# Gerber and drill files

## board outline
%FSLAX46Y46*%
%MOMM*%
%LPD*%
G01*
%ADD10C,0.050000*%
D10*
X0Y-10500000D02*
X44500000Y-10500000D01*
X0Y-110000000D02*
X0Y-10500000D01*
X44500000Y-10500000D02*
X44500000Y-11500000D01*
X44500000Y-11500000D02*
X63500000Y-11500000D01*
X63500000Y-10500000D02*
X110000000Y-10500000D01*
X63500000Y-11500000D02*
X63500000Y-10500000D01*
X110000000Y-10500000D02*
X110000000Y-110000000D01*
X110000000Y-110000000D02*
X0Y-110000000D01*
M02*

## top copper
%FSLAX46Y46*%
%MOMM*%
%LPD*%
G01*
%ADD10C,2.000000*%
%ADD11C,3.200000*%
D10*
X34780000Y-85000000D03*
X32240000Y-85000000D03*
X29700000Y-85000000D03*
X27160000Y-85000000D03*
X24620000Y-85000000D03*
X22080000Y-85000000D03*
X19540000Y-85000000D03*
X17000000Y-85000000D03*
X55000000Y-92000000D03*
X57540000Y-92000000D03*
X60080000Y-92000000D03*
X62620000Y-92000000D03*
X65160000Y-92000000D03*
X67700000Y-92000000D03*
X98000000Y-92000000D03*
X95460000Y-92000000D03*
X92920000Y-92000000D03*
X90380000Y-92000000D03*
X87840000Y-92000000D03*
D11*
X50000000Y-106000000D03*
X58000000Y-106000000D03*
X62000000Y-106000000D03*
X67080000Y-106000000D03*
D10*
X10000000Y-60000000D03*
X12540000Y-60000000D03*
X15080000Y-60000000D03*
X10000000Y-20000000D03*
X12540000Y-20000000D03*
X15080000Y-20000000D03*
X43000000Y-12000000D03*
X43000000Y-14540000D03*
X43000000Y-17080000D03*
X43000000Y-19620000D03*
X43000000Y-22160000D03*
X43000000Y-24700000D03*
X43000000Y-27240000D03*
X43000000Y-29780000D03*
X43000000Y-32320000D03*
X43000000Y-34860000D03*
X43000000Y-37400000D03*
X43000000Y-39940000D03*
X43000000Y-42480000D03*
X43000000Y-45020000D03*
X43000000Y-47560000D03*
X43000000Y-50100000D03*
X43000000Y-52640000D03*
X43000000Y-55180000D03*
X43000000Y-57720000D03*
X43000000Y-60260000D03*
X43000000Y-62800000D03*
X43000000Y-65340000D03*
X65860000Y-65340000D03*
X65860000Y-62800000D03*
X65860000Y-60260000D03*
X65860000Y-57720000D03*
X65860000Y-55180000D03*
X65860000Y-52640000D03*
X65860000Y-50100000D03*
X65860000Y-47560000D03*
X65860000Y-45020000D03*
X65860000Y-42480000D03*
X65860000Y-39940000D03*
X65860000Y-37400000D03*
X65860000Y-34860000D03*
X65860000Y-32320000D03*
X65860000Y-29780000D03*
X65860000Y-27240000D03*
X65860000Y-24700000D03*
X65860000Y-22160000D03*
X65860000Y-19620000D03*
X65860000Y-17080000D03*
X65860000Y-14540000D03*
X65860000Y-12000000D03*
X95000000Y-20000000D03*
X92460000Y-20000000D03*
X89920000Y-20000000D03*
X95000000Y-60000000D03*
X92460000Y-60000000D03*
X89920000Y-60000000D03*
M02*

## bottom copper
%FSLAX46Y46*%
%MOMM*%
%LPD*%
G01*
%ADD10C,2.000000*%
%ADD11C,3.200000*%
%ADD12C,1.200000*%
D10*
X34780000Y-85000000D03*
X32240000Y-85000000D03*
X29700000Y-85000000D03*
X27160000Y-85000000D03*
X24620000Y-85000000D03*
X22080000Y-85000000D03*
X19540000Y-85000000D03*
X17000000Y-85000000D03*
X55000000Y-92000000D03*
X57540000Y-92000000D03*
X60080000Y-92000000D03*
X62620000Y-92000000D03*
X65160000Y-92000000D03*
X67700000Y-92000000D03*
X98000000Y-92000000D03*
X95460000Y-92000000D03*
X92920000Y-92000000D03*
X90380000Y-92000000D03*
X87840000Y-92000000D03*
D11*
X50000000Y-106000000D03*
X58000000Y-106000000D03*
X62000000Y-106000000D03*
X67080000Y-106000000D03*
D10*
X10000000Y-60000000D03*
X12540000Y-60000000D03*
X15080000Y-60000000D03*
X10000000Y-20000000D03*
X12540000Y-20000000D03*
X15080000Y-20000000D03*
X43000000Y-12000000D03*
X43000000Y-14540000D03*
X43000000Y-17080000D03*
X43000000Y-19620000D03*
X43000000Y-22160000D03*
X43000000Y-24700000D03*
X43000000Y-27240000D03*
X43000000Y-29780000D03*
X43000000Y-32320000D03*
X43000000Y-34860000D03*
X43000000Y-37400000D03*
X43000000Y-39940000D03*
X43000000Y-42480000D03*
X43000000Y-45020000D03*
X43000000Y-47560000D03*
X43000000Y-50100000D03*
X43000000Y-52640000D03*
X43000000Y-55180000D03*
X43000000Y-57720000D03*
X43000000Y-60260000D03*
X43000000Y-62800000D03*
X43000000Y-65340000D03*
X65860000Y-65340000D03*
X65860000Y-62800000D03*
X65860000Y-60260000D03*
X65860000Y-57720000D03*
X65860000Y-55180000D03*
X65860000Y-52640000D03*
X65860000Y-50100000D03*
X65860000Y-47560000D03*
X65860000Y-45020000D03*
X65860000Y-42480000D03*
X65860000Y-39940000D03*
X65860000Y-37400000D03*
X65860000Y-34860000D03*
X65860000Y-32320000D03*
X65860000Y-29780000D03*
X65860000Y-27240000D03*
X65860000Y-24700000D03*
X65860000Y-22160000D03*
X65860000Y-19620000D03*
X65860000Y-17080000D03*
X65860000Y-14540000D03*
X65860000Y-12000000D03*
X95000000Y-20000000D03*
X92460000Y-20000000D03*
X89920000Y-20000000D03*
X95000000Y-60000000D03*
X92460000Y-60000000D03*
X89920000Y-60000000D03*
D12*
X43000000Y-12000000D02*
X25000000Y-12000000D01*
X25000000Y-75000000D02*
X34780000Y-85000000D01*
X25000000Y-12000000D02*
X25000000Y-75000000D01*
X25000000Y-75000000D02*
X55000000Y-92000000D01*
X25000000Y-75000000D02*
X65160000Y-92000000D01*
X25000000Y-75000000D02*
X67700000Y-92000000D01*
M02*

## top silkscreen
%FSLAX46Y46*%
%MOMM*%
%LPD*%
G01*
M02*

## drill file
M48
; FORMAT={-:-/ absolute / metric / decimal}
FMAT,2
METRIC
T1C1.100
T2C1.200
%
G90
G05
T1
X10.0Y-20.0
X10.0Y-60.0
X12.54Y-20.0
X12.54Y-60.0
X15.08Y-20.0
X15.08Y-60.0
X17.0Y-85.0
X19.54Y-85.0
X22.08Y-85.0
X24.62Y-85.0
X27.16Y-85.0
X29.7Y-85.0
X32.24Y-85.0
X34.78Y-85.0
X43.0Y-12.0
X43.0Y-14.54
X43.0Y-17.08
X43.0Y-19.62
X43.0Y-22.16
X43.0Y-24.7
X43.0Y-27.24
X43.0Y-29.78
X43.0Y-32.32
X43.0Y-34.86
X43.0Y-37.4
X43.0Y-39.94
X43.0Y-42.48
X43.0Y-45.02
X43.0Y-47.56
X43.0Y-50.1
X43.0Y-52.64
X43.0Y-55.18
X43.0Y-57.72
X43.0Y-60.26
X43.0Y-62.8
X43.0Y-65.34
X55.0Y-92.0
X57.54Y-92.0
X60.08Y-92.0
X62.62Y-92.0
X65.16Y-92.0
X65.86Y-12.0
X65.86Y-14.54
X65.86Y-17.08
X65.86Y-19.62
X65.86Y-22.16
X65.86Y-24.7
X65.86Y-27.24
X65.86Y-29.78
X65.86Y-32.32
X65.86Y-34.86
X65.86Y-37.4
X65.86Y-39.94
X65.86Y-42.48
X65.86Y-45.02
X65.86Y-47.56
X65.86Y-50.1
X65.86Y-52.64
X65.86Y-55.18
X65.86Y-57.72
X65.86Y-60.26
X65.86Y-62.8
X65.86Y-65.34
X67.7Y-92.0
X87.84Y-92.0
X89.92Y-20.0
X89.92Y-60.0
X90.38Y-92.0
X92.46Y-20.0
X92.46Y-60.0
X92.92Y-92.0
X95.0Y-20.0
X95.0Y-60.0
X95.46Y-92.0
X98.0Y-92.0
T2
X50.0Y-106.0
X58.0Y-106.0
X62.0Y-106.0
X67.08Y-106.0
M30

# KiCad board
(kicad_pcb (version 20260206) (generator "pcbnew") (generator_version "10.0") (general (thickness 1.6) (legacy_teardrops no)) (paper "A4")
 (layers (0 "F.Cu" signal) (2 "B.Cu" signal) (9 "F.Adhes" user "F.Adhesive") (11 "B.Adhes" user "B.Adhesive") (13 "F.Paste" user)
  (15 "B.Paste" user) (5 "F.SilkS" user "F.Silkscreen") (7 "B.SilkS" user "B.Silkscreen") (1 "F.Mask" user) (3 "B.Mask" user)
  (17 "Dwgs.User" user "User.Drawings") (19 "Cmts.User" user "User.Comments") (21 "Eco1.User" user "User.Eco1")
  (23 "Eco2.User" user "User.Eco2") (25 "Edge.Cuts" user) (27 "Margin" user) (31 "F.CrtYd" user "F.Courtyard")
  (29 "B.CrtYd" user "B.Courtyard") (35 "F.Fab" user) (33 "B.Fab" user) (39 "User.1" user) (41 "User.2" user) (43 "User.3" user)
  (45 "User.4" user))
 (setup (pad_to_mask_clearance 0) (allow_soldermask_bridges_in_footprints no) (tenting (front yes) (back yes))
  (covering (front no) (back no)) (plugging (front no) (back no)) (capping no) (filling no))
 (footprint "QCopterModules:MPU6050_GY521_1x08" (layer "F.Cu") (at 34.78 85 -90)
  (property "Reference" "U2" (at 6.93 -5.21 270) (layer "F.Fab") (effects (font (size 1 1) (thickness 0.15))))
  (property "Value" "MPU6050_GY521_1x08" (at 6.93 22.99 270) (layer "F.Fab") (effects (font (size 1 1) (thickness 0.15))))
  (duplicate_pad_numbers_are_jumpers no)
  (pad "1" thru_hole circle (at 0 0 270) (size 2 2) (drill 1.1) (layers "*.Cu" "*.Mask") (remove_unused_layers no) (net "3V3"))
  (pad "2" thru_hole circle (at 0 2.54 270) (size 2 2) (drill 1.1) (layers "*.Cu" "*.Mask") (remove_unused_layers no) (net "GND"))
  (pad "3" thru_hole circle (at 0 5.08 270) (size 2 2) (drill 1.1) (layers "*.Cu" "*.Mask") (remove_unused_layers no) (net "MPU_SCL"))
  (pad "4" thru_hole circle (at 0 7.62 270) (size 2 2) (drill 1.1) (layers "*.Cu" "*.Mask") (remove_unused_layers no) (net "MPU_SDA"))
  (pad "5" thru_hole circle (at 0 10.16 270) (size 2 2) (drill 1.1) (layers "*.Cu" "*.Mask") (remove_unused_layers no)
   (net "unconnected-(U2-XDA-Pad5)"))
  (pad "6" thru_hole circle (at 0 12.7 270) (size 2 2) (drill 1.1) (layers "*.Cu" "*.Mask") (remove_unused_layers no)
   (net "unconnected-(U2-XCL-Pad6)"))
  (pad "7" thru_hole circle (at 0 15.24 270) (size 2 2) (drill 1.1) (layers "*.Cu" "*.Mask") (remove_unused_layers no) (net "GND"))
  (pad "8" thru_hole circle (at 0 17.78 270) (size 2 2) (drill 1.1) (layers "*.Cu" "*.Mask") (remove_unused_layers no) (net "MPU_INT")))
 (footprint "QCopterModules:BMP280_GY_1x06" (layer "F.Cu") (at 55 92 90)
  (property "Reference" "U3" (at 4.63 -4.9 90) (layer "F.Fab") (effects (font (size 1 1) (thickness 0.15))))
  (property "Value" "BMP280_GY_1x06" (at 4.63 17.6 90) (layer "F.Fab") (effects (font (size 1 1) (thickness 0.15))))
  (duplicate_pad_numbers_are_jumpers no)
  (pad "1" thru_hole circle (at 0 0 90) (size 2 2) (drill 1.1) (layers "*.Cu" "*.Mask") (remove_unused_layers no) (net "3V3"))
  (pad "2" thru_hole circle (at 0 2.54 90) (size 2 2) (drill 1.1) (layers "*.Cu" "*.Mask") (remove_unused_layers no) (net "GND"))
  (pad "3" thru_hole circle (at 0 5.08 90) (size 2 2) (drill 1.1) (layers "*.Cu" "*.Mask") (remove_unused_layers no) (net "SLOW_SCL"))
  (pad "4" thru_hole circle (at 0 7.62 90) (size 2 2) (drill 1.1) (layers "*.Cu" "*.Mask") (remove_unused_layers no) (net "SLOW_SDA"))
  (pad "5" thru_hole circle (at 0 10.16 90) (size 2 2) (drill 1.1) (layers "*.Cu" "*.Mask") (remove_unused_layers no) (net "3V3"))
  (pad "6" thru_hole circle (at 0 12.7 90) (size 2 2) (drill 1.1) (layers "*.Cu" "*.Mask") (remove_unused_layers no) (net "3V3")))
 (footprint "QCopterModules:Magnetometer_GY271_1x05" (layer "F.Cu") (at 98 92 -90)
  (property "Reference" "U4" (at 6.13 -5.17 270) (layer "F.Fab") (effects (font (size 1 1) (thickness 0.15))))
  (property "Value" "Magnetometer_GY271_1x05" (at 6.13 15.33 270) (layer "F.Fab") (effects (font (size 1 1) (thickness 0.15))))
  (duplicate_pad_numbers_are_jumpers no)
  (pad "1" thru_hole circle (at 0 0 270) (size 2 2) (drill 1.1) (layers "*.Cu" "*.Mask") (remove_unused_layers no) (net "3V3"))
  (pad "2" thru_hole circle (at 0 2.54 270) (size 2 2) (drill 1.1) (layers "*.Cu" "*.Mask") (remove_unused_layers no) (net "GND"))
  (pad "3" thru_hole circle (at 0 5.08 270) (size 2 2) (drill 1.1) (layers "*.Cu" "*.Mask") (remove_unused_layers no) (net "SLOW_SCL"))
  (pad "4" thru_hole circle (at 0 7.62 270) (size 2 2) (drill 1.1) (layers "*.Cu" "*.Mask") (remove_unused_layers no) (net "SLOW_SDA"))
  (pad "5" thru_hole circle (at 0 10.16 270) (size 2 2) (drill 1.1) (layers "*.Cu" "*.Mask") (remove_unused_layers no) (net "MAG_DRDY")))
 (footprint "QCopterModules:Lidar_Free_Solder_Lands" (layer "F.Cu") (at 50 106)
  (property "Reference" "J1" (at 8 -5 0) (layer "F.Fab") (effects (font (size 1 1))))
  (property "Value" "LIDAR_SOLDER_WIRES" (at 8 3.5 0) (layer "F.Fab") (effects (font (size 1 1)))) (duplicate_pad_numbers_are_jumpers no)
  (pad "1" thru_hole circle (at 0 0) (size 3.2 3.2) (drill 1.2) (layers "*.Cu" "*.Mask") (remove_unused_layers no) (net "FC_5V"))
  (pad "2" thru_hole circle (at 8 0) (size 3.2 3.2) (drill 1.2) (layers "*.Cu" "*.Mask") (remove_unused_layers no) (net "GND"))
  (pad "3" thru_hole circle (at 12 0) (size 3.2 3.2) (drill 1.2) (layers "*.Cu" "*.Mask") (remove_unused_layers no) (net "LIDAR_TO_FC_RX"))
  (pad "4" thru_hole circle (at 17.08 0) (size 3.2 3.2) (drill 1.2) (layers "*.Cu" "*.Mask") (remove_unused_layers no)
   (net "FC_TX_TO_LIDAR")))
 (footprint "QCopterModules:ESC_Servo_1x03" (layer "F.Cu") (at 10 60 90)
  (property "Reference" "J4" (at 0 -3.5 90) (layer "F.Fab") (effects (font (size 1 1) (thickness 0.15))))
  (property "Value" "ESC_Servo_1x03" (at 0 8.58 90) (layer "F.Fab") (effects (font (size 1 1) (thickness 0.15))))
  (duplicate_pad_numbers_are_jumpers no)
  (pad "1" thru_hole circle (at 0 0 90) (size 2 2) (drill 1.1) (layers "*.Cu" "*.Mask") (remove_unused_layers no) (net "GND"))
  (pad "2" thru_hole circle (at 0 2.54 90) (size 2 2) (drill 1.1) (layers "*.Cu" "*.Mask") (remove_unused_layers no) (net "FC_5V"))
  (pad "3" thru_hole circle (at 0 5.08 90) (size 2 2) (drill 1.1) (layers "*.Cu" "*.Mask") (remove_unused_layers no) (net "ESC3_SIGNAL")))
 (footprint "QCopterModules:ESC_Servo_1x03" (layer "F.Cu") (at 10 20 90)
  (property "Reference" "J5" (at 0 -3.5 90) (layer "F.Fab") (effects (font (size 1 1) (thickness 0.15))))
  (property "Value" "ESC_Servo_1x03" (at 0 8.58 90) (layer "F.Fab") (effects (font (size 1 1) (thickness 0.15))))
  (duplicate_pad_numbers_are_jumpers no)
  (pad "1" thru_hole circle (at 0 0 90) (size 2 2) (drill 1.1) (layers "*.Cu" "*.Mask") (remove_unused_layers no) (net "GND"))
  (pad "2" thru_hole circle (at 0 2.54 90) (size 2 2) (drill 1.1) (layers "*.Cu" "*.Mask") (remove_unused_layers no)
   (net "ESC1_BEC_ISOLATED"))
  (pad "3" thru_hole circle (at 0 5.08 90) (size 2 2) (drill 1.1) (layers "*.Cu" "*.Mask") (remove_unused_layers no) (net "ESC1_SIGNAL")))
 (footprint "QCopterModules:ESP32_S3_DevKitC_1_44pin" (layer "F.Cu") (at 43 12)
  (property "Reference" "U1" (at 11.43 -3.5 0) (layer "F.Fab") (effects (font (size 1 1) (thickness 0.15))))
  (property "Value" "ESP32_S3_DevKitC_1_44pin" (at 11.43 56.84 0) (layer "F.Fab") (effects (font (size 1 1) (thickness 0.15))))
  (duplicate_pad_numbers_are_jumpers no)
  (pad "1" thru_hole circle (at 0 0) (size 2 2) (drill 1.1) (layers "*.Cu" "*.Mask") (remove_unused_layers no) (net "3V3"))
  (pad "2" thru_hole circle (at 0 2.54) (size 2 2) (drill 1.1) (layers "*.Cu" "*.Mask") (remove_unused_layers no))
  (pad "3" thru_hole circle (at 0 5.08) (size 2 2) (drill 1.1) (layers "*.Cu" "*.Mask") (remove_unused_layers no)
   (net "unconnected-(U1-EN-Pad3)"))
  (pad "4" thru_hole circle (at 0 7.62) (size 2 2) (drill 1.1) (layers "*.Cu" "*.Mask") (remove_unused_layers no) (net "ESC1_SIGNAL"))
  (pad "5" thru_hole circle (at 0 10.16) (size 2 2) (drill 1.1) (layers "*.Cu" "*.Mask") (remove_unused_layers no)
   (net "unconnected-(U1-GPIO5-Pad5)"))
  (pad "6" thru_hole circle (at 0 12.7) (size 2 2) (drill 1.1) (layers "*.Cu" "*.Mask") (remove_unused_layers no)
   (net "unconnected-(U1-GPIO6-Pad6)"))
  (pad "7" thru_hole circle (at 0 15.24) (size 2 2) (drill 1.1) (layers "*.Cu" "*.Mask") (remove_unused_layers no)
   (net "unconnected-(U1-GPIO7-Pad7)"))
  (pad "8" thru_hole circle (at 0 17.78) (size 2 2) (drill 1.1) (layers "*.Cu" "*.Mask") (remove_unused_layers no) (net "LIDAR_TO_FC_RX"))
  (pad "9" thru_hole circle (at 0 20.32) (size 2 2) (drill 1.1) (layers "*.Cu" "*.Mask") (remove_unused_layers no) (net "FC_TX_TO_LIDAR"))
  (pad "10" thru_hole circle (at 0 22.86) (size 2 2) (drill 1.1) (layers "*.Cu" "*.Mask") (remove_unused_layers no)
   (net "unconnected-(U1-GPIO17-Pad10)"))
  (pad "11" thru_hole circle (at 0 25.4) (size 2 2) (drill 1.1) (layers "*.Cu" "*.Mask") (remove_unused_layers no) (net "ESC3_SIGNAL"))
  (pad "12" thru_hole circle (at 0 27.94) (size 2 2) (drill 1.1) (layers "*.Cu" "*.Mask") (remove_unused_layers no)
   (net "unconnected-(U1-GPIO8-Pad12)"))
  (pad "13" thru_hole circle (at 0 30.48) (size 2 2) (drill 1.1) (layers "*.Cu" "*.Mask") (remove_unused_layers no)
   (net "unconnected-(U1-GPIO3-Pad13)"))
  (pad "14" thru_hole circle (at 0 33.02) (size 2 2) (drill 1.1) (layers "*.Cu" "*.Mask") (remove_unused_layers no)
   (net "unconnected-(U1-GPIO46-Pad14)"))
  (pad "15" thru_hole circle (at 0 35.56) (size 2 2) (drill 1.1) (layers "*.Cu" "*.Mask") (remove_unused_layers no)
   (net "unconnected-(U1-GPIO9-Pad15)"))
  (pad "16" thru_hole circle (at 0 38.1) (size 2 2) (drill 1.1) (layers "*.Cu" "*.Mask") (remove_unused_layers no)
   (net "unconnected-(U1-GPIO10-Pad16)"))
  (pad "17" thru_hole circle (at 0 40.64) (size 2 2) (drill 1.1) (layers "*.Cu" "*.Mask") (remove_unused_layers no)
   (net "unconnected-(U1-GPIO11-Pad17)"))
  (pad "18" thru_hole circle (at 0 43.18) (size 2 2) (drill 1.1) (layers "*.Cu" "*.Mask") (remove_unused_layers no) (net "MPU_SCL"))
  (pad "19" thru_hole circle (at 0 45.72) (size 2 2) (drill 1.1) (layers "*.Cu" "*.Mask") (remove_unused_layers no) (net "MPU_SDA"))
  (pad "20" thru_hole circle (at 0 48.26) (size 2 2) (drill 1.1) (layers "*.Cu" "*.Mask") (remove_unused_layers no) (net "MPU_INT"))
  (pad "21" thru_hole circle (at 0 50.8) (size 2 2) (drill 1.1) (layers "*.Cu" "*.Mask") (remove_unused_layers no) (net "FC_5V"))
  (pad "22" thru_hole circle (at 0 53.34) (size 2 2) (drill 1.1) (layers "*.Cu" "*.Mask") (remove_unused_layers no) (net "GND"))
  (pad "23" thru_hole circle (at 22.86 53.34) (size 2 2) (drill 1.1) (layers "*.Cu" "*.Mask") (remove_unused_layers no) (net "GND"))
  (pad "24" thru_hole circle (at 22.86 50.8) (size 2 2) (drill 1.1) (layers "*.Cu" "*.Mask") (remove_unused_layers no) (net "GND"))
  (pad "25" thru_hole circle (at 22.86 48.26) (size 2 2) (drill 1.1) (layers "*.Cu" "*.Mask") (remove_unused_layers no)
   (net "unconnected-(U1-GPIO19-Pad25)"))
  (pad "26" thru_hole circle (at 22.86 45.72) (size 2 2) (drill 1.1) (layers "*.Cu" "*.Mask") (remove_unused_layers no)
   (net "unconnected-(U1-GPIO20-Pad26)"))
  (pad "27" thru_hole circle (at 22.86 43.18) (size 2 2) (drill 1.1) (layers "*.Cu" "*.Mask") (remove_unused_layers no) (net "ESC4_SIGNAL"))
  (pad "28" thru_hole circle (at 22.86 40.64) (size 2 2) (drill 1.1) (layers "*.Cu" "*.Mask") (remove_unused_layers no)
   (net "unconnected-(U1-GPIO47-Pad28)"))
  (pad "29" thru_hole circle (at 22.86 38.1) (size 2 2) (drill 1.1) (layers "*.Cu" "*.Mask") (remove_unused_layers no)
   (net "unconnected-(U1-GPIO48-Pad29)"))
  (pad "30" thru_hole circle (at 22.86 35.56) (size 2 2) (drill 1.1) (layers "*.Cu" "*.Mask") (remove_unused_layers no)
   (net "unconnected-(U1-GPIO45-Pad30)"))
  (pad "31" thru_hole circle (at 22.86 33.02) (size 2 2) (drill 1.1) (layers "*.Cu" "*.Mask") (remove_unused_layers no)
   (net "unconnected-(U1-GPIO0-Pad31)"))
  (pad "32" thru_hole circle (at 22.86 30.48) (size 2 2) (drill 1.1) (layers "*.Cu" "*.Mask") (remove_unused_layers no)
   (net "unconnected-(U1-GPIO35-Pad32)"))
  (pad "33" thru_hole circle (at 22.86 27.94) (size 2 2) (drill 1.1) (layers "*.Cu" "*.Mask") (remove_unused_layers no)
   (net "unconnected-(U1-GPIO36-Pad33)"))
  (pad "34" thru_hole circle (at 22.86 25.4) (size 2 2) (drill 1.1) (layers "*.Cu" "*.Mask") (remove_unused_layers no)
   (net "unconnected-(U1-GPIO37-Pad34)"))
  (pad "35" thru_hole circle (at 22.86 22.86) (size 2 2) (drill 1.1) (layers "*.Cu" "*.Mask") (remove_unused_layers no)
   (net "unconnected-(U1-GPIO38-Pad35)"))
  (pad "36" thru_hole circle (at 22.86 20.32) (size 2 2) (drill 1.1) (layers "*.Cu" "*.Mask") (remove_unused_layers no) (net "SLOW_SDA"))
  (pad "37" thru_hole circle (at 22.86 17.78) (size 2 2) (drill 1.1) (layers "*.Cu" "*.Mask") (remove_unused_layers no) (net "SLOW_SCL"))
  (pad "38" thru_hole circle (at 22.86 15.24) (size 2 2) (drill 1.1) (layers "*.Cu" "*.Mask") (remove_unused_layers no) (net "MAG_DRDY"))
  (pad "39" thru_hole circle (at 22.86 12.7) (size 2 2) (drill 1.1) (layers "*.Cu" "*.Mask") (remove_unused_layers no)
   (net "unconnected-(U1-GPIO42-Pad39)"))
  (pad "40" thru_hole circle (at 22.86 10.16) (size 2 2) (drill 1.1) (layers "*.Cu" "*.Mask") (remove_unused_layers no) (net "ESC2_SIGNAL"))
  (pad "41" thru_hole circle (at 22.86 7.62) (size 2 2) (drill 1.1) (layers "*.Cu" "*.Mask") (remove_unused_layers no)
   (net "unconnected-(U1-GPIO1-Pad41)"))
  (pad "42" thru_hole circle (at 22.86 5.08) (size 2 2) (drill 1.1) (layers "*.Cu" "*.Mask") (remove_unused_layers no)
   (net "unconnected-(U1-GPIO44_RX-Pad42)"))
  (pad "43" thru_hole circle (at 22.86 2.54) (size 2 2) (drill 1.1) (layers "*.Cu" "*.Mask") (remove_unused_layers no)
   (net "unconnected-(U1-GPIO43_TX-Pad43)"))
  (pad "44" thru_hole circle (at 22.86 0) (size 2 2) (drill 1.1) (layers "*.Cu" "*.Mask") (remove_unused_layers no) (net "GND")))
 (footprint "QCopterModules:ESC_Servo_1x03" (layer "F.Cu") (at 95 20 -90)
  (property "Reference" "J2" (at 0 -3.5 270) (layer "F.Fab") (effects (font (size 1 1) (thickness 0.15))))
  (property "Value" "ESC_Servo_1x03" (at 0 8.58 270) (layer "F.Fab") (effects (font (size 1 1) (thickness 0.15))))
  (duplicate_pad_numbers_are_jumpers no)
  (pad "1" thru_hole circle (at 0 0 270) (size 2 2) (drill 1.1) (layers "*.Cu" "*.Mask") (remove_unused_layers no) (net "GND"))
  (pad "2" thru_hole circle (at 0 2.54 270) (size 2 2) (drill 1.1) (layers "*.Cu" "*.Mask") (remove_unused_layers no)
   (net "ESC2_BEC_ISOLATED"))
  (pad "3" thru_hole circle (at 0 5.08 270) (size 2 2) (drill 1.1) (layers "*.Cu" "*.Mask") (remove_unused_layers no) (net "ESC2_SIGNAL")))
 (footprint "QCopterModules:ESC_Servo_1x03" (layer "F.Cu") (at 95 60 -90)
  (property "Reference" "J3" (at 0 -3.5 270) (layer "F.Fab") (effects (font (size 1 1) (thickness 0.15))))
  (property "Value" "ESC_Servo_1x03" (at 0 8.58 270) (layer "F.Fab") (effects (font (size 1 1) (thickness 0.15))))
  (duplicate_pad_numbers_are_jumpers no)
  (pad "1" thru_hole circle (at 0 0 270) (size 2 2) (drill 1.1) (layers "*.Cu" "*.Mask") (remove_unused_layers no) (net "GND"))
  (pad "2" thru_hole circle (at 0 2.54 270) (size 2 2) (drill 1.1) (layers "*.Cu" "*.Mask") (remove_unused_layers no)
   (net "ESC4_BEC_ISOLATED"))
  (pad "3" thru_hole circle (at 0 5.08 270) (size 2 2) (drill 1.1) (layers "*.Cu" "*.Mask") (remove_unused_layers no) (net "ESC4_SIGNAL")))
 (gr_line (start 0 10.5) (end 44.5 10.5) (stroke (width 0.05) (type default)) (layer "Edge.Cuts"))
 (gr_line (start 0 110) (end 0 10.5) (stroke (width 0.05) (type default)) (layer "Edge.Cuts"))
 (gr_line (start 44.5 10.5) (end 44.5 11.5) (stroke (width 0.05) (type default)) (layer "Edge.Cuts"))
 (gr_line (start 44.5 11.5) (end 63.5 11.5) (stroke (width 0.05) (type default)) (layer "Edge.Cuts"))
 (gr_line (start 63.5 10.5) (end 110 10.5) (stroke (width 0.05) (type default)) (layer "Edge.Cuts"))
 (gr_line (start 63.5 11.5) (end 63.5 10.5) (stroke (width 0.05) (type default)) (layer "Edge.Cuts"))
 (gr_line (start 110 10.5) (end 110 110) (stroke (width 0.05) (type default)) (layer "Edge.Cuts"))
 (gr_line (start 110 110) (end 0 110) (stroke (width 0.05) (type default)) (layer "Edge.Cuts"))
 (segment (start 43 12) (end 25 12) (width 1.2) (layer "B.Cu") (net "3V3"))
 (segment (start 25 75) (end 34.78 85) (width 1.2) (layer "B.Cu") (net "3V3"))
 (segment (start 25 12) (end 25 75) (width 1.2) (layer "B.Cu") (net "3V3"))
 (segment (start 25 75) (end 55 92) (width 1.2) (layer "B.Cu") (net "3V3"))
 (segment (start 25 75) (end 65.16 92) (width 1.2) (layer "B.Cu") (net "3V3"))
 (segment (start 25 75) (end 67.7 92) (width 1.2) (layer "B.Cu") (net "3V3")))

